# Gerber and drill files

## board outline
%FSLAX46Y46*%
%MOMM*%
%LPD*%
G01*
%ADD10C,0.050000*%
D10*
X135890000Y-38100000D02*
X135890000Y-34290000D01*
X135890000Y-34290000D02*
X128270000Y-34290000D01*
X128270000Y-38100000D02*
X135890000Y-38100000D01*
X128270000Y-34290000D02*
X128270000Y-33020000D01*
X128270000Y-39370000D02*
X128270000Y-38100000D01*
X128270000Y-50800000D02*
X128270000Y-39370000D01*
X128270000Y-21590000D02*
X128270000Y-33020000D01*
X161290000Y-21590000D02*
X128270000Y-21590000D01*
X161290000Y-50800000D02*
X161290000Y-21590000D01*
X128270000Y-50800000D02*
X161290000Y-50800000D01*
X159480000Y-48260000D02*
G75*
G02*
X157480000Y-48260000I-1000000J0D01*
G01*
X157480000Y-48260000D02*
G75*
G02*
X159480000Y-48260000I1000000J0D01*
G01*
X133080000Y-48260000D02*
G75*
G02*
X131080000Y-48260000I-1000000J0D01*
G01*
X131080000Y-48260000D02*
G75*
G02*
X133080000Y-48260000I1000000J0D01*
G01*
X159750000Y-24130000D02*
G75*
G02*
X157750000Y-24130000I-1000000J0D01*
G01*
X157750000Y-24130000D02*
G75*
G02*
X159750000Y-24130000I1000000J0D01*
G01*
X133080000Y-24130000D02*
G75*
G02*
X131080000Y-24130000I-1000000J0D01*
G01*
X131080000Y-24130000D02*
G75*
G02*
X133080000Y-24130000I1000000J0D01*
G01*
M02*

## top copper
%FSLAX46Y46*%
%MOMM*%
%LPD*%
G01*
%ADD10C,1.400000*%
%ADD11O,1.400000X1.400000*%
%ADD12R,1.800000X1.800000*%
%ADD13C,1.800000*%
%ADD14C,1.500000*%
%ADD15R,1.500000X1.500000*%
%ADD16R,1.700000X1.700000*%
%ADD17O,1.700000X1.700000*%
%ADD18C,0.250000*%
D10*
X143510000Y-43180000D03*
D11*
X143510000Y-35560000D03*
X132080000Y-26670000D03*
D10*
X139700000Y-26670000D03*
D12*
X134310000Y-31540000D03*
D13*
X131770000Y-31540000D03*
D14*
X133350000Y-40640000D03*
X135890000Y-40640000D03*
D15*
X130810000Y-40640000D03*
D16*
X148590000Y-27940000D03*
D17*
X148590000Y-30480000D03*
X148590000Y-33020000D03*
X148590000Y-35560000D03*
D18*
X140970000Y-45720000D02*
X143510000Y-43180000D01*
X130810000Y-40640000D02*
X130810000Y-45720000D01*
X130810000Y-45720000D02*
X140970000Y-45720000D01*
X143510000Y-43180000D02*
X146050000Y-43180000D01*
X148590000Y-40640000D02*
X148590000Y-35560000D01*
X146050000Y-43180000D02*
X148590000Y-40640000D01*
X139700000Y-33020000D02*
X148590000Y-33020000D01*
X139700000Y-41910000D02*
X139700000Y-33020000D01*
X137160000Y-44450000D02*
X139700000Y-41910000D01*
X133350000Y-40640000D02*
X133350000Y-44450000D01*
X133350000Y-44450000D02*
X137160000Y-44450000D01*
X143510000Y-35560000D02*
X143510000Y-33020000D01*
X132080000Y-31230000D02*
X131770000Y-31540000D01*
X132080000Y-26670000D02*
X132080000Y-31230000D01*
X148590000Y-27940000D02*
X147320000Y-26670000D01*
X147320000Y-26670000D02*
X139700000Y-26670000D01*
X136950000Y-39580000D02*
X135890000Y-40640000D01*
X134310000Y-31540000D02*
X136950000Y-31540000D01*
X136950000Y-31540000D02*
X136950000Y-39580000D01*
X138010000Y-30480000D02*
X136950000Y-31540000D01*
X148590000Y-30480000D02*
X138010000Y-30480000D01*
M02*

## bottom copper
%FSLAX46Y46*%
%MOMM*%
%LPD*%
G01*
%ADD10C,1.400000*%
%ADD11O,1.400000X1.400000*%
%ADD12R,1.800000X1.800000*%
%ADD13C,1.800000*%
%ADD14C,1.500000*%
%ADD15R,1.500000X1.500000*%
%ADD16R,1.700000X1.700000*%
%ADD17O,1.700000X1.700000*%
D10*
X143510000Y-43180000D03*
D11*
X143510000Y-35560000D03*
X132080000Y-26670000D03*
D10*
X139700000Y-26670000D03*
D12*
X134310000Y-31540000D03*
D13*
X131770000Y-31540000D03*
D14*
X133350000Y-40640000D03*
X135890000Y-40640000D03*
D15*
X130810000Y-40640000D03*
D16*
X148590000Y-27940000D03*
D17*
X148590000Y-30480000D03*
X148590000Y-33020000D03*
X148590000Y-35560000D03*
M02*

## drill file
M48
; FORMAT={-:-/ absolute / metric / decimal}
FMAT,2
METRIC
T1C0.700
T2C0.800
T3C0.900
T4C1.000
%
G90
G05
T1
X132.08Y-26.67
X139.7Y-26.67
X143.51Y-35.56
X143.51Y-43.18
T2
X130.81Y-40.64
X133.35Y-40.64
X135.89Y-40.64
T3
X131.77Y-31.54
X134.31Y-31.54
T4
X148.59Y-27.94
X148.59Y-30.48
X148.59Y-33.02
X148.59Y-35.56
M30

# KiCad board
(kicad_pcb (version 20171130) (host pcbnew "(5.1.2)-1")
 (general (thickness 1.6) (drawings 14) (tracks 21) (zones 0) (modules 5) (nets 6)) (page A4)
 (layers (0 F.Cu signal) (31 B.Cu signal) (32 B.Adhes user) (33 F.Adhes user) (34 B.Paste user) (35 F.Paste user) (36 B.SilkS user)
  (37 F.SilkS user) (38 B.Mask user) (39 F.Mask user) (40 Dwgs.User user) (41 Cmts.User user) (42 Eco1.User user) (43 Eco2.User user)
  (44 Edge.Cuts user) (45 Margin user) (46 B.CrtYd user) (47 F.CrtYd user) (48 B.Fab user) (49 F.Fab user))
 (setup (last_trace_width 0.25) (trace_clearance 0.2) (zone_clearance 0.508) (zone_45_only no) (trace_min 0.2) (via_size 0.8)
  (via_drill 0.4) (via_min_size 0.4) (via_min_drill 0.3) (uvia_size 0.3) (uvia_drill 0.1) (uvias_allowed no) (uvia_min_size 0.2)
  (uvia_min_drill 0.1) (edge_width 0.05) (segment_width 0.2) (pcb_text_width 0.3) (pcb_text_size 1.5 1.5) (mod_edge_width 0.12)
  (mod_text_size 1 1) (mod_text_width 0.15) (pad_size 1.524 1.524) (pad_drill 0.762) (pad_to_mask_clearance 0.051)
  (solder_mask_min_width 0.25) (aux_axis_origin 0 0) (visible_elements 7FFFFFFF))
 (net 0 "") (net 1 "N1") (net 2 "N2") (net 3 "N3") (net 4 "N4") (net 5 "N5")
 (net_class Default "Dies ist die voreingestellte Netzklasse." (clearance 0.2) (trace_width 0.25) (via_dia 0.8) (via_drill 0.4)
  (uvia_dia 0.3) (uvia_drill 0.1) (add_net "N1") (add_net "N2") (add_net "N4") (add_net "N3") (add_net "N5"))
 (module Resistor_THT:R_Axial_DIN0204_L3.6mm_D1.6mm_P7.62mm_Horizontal (layer F.Cu) (at 143.51 43.18 90)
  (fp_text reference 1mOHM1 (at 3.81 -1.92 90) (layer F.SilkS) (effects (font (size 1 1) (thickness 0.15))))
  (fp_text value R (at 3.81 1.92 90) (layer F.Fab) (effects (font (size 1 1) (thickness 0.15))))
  (pad 1 thru_hole circle (at 0 0 90) (size 1.4 1.4) (drill 0.7) (layers *.Cu *.Mask) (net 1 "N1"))
  (pad 2 thru_hole oval (at 7.62 0 90) (size 1.4 1.4) (drill 0.7) (layers *.Cu *.Mask) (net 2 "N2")))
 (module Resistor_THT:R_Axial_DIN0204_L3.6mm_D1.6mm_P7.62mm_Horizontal (layer F.Cu) (at 139.7 26.67 180)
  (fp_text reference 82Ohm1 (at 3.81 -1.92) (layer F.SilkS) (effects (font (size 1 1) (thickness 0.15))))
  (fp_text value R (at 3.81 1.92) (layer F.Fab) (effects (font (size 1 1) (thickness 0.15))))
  (pad 2 thru_hole oval (at 7.62 0 180) (size 1.4 1.4) (drill 0.7) (layers *.Cu *.Mask) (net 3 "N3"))
  (pad 1 thru_hole circle (at 0 0 180) (size 1.4 1.4) (drill 0.7) (layers *.Cu *.Mask) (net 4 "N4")))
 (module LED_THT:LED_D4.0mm (layer F.Cu) (at 134.31 31.54 180)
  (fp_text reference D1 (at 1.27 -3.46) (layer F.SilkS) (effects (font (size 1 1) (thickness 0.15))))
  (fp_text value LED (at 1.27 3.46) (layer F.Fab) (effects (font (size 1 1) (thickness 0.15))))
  (pad 1 thru_hole rect (at 0 0 180) (size 1.8 1.8) (drill 0.9) (layers *.Cu *.Mask) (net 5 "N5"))
  (pad 2 thru_hole circle (at 2.54 0 180) (size 1.8 1.8) (drill 0.9) (layers *.Cu *.Mask) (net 3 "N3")))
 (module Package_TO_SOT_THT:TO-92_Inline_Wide (layer F.Cu) (at 130.81 40.64)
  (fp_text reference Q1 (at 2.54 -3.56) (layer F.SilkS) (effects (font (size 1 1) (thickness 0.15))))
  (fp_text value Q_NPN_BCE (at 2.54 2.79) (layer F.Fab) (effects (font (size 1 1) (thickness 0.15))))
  (pad 2 thru_hole circle (at 2.54 0 90) (size 1.5 1.5) (drill 0.8) (layers *.Cu *.Mask) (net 2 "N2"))
  (pad 3 thru_hole circle (at 5.08 0 90) (size 1.5 1.5) (drill 0.8) (layers *.Cu *.Mask) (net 5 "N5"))
  (pad 1 thru_hole rect (at 0 0 90) (size 1.5 1.5) (drill 0.8) (layers *.Cu *.Mask) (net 1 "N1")))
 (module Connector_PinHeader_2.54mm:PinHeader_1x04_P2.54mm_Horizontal (layer F.Cu) (at 148.59 27.94)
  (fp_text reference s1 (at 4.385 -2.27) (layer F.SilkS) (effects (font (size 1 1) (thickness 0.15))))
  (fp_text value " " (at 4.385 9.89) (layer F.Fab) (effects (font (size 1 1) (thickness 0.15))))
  (pad 1 thru_hole rect (at 0 0) (size 1.7 1.7) (drill 1) (layers *.Cu *.Mask) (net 4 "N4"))
  (pad 2 thru_hole oval (at 0 2.54) (size 1.7 1.7) (drill 1) (layers *.Cu *.Mask) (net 5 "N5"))
  (pad 3 thru_hole oval (at 0 5.08) (size 1.7 1.7) (drill 1) (layers *.Cu *.Mask) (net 2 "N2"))
  (pad 4 thru_hole oval (at 0 7.62) (size 1.7 1.7) (drill 1) (layers *.Cu *.Mask) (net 1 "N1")))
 (gr_line (start 135.89 38.1) (end 135.89 34.29) (layer Edge.Cuts) (width 0.05))
 (gr_line (start 135.89 34.29) (end 128.27 34.29) (layer Edge.Cuts) (width 0.05))
 (gr_line (start 128.27 38.1) (end 135.89 38.1) (layer Edge.Cuts) (width 0.05))
 (gr_line (start 128.27 34.29) (end 128.27 33.02) (layer Edge.Cuts) (width 0.05))
 (gr_line (start 128.27 39.37) (end 128.27 38.1) (layer Edge.Cuts) (width 0.05))
 (gr_line (start 128.27 50.8) (end 128.27 39.37) (layer Edge.Cuts) (width 0.05))
 (gr_line (start 128.27 21.59) (end 128.27 33.02) (layer Edge.Cuts) (width 0.05))
 (gr_line (start 161.29 21.59) (end 128.27 21.59) (layer Edge.Cuts) (width 0.05))
 (gr_line (start 161.29 50.8) (end 161.29 21.59) (layer Edge.Cuts) (width 0.05))
 (gr_line (start 128.27 50.8) (end 161.29 50.8) (layer Edge.Cuts) (width 0.05))
 (gr_circle (center 158.48 48.26) (end 159.48 48.26) (layer Edge.Cuts) (width 0.05))
 (gr_circle (center 132.08 48.26) (end 133.08 48.26) (layer Edge.Cuts) (width 0.05))
 (gr_circle (center 158.75 24.13) (end 159.75 24.13) (layer Edge.Cuts) (width 0.05))
 (gr_circle (center 132.08 24.13) (end 133.08 24.13) (layer Edge.Cuts) (width 0.05))
 (segment (start 140.97 45.72) (end 143.51 43.18) (width 0.25) (layer F.Cu) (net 1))
 (segment (start 130.81 40.64) (end 130.81 45.72) (width 0.25) (layer F.Cu) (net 1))
 (segment (start 130.81 45.72) (end 140.97 45.72) (width 0.25) (layer F.Cu) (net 1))
 (segment (start 143.51 43.18) (end 146.05 43.18) (width 0.25) (layer F.Cu) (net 1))
 (segment (start 148.59 40.64) (end 148.59 35.56) (width 0.25) (layer F.Cu) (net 1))
 (segment (start 146.05 43.18) (end 148.59 40.64) (width 0.25) (layer F.Cu) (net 1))
 (segment (start 139.7 33.02) (end 148.59 33.02) (width 0.25) (layer F.Cu) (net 2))
 (segment (start 139.7 41.91) (end 139.7 33.02) (width 0.25) (layer F.Cu) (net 2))
 (segment (start 137.16 44.45) (end 139.7 41.91) (width 0.25) (layer F.Cu) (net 2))
 (segment (start 133.35 40.64) (end 133.35 44.45) (width 0.25) (layer F.Cu) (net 2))
 (segment (start 133.35 44.45) (end 137.16 44.45) (width 0.25) (layer F.Cu) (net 2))
 (segment (start 143.51 35.56) (end 143.51 33.02) (width 0.25) (layer F.Cu) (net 2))
 (segment (start 132.08 31.23) (end 131.77 31.54) (width 0.25) (layer F.Cu) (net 3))
 (segment (start 132.08 26.67) (end 132.08 31.23) (width 0.25) (layer F.Cu) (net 3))
 (segment (start 148.59 27.94) (end 147.32 26.67) (width 0.25) (layer F.Cu) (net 4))
 (segment (start 147.32 26.67) (end 139.7 26.67) (width 0.25) (layer F.Cu) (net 4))
 (segment (start 136.95 39.58) (end 135.89 40.64) (width 0.25) (layer F.Cu) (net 5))
 (segment (start 134.31 31.54) (end 136.95 31.54) (width 0.25) (layer F.Cu) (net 5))
 (segment (start 136.95 31.54) (end 136.95 39.58) (width 0.25) (layer F.Cu) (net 5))
 (segment (start 138.01 30.48) (end 136.95 31.54) (width 0.25) (layer F.Cu) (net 5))
 (segment (start 148.59 30.48) (end 138.01 30.48) (width 0.25) (layer F.Cu) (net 5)))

